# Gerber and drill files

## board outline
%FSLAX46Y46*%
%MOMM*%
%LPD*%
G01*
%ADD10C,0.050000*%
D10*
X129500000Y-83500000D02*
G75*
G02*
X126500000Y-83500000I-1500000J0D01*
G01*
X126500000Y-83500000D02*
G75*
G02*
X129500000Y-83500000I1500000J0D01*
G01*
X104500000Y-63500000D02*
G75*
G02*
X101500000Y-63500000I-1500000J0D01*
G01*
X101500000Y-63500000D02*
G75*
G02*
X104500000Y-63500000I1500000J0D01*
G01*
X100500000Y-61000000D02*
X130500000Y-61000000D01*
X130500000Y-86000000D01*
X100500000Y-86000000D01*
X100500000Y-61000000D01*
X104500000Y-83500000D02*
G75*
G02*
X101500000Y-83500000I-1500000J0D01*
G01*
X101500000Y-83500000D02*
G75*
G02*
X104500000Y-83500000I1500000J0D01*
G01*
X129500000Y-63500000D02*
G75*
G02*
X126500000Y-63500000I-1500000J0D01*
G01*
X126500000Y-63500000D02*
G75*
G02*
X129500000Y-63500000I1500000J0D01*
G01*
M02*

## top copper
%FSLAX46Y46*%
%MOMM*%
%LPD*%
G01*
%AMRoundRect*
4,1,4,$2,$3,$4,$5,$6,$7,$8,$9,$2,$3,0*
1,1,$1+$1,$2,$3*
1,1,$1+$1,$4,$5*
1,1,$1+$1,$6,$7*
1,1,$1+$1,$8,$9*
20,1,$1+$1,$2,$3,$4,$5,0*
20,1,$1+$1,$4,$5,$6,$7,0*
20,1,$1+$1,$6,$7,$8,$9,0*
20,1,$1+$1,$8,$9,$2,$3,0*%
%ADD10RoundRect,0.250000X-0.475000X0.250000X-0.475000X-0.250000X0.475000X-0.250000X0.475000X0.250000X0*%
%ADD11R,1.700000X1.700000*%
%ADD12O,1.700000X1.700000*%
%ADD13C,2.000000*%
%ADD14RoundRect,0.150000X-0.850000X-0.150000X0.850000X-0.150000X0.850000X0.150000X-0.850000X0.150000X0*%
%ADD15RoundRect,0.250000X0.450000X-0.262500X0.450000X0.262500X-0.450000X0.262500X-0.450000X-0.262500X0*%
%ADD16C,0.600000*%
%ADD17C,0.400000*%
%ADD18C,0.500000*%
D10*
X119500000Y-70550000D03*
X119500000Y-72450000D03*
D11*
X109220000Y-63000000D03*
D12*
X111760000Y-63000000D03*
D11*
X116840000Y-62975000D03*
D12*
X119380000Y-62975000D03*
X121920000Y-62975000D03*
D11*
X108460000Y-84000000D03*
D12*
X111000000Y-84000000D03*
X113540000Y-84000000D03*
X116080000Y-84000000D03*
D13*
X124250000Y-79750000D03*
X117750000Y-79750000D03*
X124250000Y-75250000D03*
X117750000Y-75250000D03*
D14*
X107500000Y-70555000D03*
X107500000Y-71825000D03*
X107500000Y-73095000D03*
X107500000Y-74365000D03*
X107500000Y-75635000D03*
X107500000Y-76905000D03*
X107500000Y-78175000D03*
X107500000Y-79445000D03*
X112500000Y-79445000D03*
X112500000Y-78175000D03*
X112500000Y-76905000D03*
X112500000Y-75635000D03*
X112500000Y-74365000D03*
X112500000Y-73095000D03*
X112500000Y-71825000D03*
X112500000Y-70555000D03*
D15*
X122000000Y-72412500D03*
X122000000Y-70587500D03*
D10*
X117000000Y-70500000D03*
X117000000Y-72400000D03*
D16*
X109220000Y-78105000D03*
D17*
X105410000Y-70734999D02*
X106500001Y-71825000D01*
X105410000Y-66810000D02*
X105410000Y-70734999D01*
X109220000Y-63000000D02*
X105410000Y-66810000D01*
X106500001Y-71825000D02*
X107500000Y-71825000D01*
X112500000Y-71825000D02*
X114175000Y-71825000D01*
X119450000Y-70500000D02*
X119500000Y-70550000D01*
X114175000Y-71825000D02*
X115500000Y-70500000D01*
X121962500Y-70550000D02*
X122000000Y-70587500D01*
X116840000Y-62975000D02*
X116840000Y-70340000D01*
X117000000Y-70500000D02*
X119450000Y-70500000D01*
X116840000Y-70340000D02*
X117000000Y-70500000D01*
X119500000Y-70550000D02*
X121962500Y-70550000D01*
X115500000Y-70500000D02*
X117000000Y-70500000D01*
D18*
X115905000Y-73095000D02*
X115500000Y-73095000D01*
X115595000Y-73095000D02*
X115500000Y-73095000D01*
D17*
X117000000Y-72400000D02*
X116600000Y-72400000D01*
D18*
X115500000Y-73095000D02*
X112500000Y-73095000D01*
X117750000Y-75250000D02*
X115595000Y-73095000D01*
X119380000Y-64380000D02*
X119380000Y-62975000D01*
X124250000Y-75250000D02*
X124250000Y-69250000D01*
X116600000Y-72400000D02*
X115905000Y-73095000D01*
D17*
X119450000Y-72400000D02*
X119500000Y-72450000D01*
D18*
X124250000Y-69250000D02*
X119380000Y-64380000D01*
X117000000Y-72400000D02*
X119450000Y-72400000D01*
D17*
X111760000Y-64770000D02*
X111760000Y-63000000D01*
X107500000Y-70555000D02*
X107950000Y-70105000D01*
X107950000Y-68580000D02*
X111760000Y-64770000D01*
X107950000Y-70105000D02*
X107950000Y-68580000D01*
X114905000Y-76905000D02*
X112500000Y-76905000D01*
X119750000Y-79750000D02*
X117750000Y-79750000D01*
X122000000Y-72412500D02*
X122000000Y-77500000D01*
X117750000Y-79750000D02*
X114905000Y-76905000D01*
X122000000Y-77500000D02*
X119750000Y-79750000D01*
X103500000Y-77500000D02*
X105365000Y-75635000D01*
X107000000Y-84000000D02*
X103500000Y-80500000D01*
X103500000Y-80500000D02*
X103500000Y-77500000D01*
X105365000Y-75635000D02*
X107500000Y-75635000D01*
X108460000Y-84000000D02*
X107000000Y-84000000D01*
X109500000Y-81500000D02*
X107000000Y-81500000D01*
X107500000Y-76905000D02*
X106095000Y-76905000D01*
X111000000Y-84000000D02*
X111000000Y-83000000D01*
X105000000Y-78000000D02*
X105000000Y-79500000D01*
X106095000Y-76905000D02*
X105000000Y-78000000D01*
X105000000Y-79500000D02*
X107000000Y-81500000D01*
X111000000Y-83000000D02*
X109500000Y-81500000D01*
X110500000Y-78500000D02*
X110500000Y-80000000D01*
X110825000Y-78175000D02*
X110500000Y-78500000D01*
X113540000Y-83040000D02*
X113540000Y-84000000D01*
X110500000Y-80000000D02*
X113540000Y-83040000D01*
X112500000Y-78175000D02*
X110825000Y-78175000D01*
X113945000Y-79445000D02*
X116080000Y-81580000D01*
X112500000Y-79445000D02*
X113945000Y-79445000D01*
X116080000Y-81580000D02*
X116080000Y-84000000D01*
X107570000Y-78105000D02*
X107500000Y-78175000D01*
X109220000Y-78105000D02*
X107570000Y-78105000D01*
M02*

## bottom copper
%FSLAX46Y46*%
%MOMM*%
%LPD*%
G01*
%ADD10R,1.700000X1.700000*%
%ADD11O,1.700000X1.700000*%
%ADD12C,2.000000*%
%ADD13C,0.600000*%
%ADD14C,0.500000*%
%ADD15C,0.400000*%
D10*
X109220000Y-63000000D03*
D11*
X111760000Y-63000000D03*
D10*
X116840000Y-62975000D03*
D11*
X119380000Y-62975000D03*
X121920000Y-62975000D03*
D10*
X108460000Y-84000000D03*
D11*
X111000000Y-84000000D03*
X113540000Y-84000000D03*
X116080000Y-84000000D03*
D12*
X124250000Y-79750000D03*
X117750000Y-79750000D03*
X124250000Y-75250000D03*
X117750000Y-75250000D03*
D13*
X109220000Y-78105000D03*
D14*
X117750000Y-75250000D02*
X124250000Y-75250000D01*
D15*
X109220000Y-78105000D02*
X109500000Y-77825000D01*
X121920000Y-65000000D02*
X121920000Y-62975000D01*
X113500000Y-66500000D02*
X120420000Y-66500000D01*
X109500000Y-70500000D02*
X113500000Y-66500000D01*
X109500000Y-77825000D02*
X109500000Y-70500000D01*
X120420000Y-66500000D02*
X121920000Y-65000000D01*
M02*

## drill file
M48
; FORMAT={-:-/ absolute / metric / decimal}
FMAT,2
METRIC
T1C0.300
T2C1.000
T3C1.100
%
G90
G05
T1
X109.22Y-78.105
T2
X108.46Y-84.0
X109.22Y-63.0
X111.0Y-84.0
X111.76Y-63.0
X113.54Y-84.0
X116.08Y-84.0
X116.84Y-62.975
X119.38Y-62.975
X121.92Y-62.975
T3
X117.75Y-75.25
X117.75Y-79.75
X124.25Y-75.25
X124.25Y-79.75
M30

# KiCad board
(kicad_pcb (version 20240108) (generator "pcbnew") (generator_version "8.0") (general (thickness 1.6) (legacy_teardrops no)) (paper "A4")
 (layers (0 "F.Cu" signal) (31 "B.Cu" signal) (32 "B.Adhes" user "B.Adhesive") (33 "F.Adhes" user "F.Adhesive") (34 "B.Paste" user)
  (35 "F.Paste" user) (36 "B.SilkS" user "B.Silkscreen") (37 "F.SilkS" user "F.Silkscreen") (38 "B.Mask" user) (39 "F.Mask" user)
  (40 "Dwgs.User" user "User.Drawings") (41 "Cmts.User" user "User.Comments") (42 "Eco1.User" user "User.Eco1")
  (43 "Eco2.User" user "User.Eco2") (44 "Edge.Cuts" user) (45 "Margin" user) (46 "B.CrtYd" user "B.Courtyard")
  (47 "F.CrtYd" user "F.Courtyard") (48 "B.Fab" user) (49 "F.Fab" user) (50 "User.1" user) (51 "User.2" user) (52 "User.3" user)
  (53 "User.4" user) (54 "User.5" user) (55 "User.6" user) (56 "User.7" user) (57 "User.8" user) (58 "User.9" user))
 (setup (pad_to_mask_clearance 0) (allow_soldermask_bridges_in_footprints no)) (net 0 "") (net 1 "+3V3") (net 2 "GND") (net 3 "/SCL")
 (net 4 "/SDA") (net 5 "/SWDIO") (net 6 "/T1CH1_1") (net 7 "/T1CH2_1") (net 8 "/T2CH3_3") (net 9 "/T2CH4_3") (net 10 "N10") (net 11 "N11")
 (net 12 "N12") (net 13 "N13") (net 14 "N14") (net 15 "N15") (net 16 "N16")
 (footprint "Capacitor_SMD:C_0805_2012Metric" (layer "F.Cu") (at 119.5 71.5 -90)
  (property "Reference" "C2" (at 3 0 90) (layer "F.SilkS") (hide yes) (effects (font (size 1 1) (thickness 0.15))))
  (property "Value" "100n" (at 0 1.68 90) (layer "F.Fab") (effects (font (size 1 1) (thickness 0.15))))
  (pad "1" smd roundrect (at -0.95 0 270) (size 1 1.45) (layers "F.Cu" "F.Paste" "F.Mask") (roundrect_rratio 0.25) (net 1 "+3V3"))
  (pad "2" smd roundrect (at 0.95 0 270) (size 1 1.45) (layers "F.Cu" "F.Paste" "F.Mask") (roundrect_rratio 0.25) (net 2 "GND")))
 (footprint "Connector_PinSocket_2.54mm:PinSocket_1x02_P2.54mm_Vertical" (layer "F.Cu") (at 109.22 63 90)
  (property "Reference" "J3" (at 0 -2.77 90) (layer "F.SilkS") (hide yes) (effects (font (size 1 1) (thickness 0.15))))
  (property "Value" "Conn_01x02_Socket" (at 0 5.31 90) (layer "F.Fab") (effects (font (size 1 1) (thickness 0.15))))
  (pad "1" thru_hole rect (at 0 0 90) (size 1.7 1.7) (drill 1) (layers "*.Cu" "*.Mask") (remove_unused_layers no) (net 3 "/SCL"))
  (pad "2" thru_hole oval (at 0 2.54 90) (size 1.7 1.7) (drill 1) (layers "*.Cu" "*.Mask") (remove_unused_layers no) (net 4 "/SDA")))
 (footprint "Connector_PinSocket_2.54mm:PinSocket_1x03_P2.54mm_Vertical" (layer "F.Cu") (at 116.84 62.975 90)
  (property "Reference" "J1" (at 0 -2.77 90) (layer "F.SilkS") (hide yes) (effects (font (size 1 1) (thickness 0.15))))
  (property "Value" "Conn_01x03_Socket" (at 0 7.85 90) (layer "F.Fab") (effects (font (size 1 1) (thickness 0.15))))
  (pad "1" thru_hole rect (at 0 0 90) (size 1.7 1.7) (drill 1) (layers "*.Cu" "*.Mask") (remove_unused_layers no) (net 1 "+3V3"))
  (pad "2" thru_hole oval (at 0 2.54 90) (size 1.7 1.7) (drill 1) (layers "*.Cu" "*.Mask") (remove_unused_layers no) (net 2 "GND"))
  (pad "3" thru_hole oval (at 0 5.08 90) (size 1.7 1.7) (drill 1) (layers "*.Cu" "*.Mask") (remove_unused_layers no) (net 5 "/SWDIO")))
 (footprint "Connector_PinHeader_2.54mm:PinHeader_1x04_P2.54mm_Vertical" (layer "F.Cu") (at 108.46 84 90)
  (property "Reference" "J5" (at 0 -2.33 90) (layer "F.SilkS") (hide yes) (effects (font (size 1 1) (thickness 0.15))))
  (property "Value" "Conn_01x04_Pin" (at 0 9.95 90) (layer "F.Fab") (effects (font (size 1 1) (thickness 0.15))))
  (pad "1" thru_hole rect (at 0 0 90) (size 1.7 1.7) (drill 1) (layers "*.Cu" "*.Mask") (remove_unused_layers no) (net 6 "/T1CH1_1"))
  (pad "2" thru_hole oval (at 0 2.54 90) (size 1.7 1.7) (drill 1) (layers "*.Cu" "*.Mask") (remove_unused_layers no) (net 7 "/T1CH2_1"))
  (pad "3" thru_hole oval (at 0 5.08 90) (size 1.7 1.7) (drill 1) (layers "*.Cu" "*.Mask") (remove_unused_layers no) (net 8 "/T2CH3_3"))
  (pad "4" thru_hole oval (at 0 7.62 90) (size 1.7 1.7) (drill 1) (layers "*.Cu" "*.Mask") (remove_unused_layers no) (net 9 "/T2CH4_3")))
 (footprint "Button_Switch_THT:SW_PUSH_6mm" (layer "F.Cu") (at 124.25 79.75 180)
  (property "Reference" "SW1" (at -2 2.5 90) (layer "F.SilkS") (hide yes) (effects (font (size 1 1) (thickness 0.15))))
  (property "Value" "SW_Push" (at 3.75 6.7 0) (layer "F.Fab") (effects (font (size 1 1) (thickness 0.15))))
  (pad "1" thru_hole circle (at 0 0 270) (size 2 2) (drill 1.1) (layers "*.Cu" "*.Mask") (remove_unused_layers no) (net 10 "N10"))
  (pad "1" thru_hole circle (at 6.5 0 270) (size 2 2) (drill 1.1) (layers "*.Cu" "*.Mask") (remove_unused_layers no) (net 10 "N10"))
  (pad "2" thru_hole circle (at 0 4.5 270) (size 2 2) (drill 1.1) (layers "*.Cu" "*.Mask") (remove_unused_layers no) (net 2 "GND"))
  (pad "2" thru_hole circle (at 6.5 4.5 270) (size 2 2) (drill 1.1) (layers "*.Cu" "*.Mask") (remove_unused_layers no) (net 2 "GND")))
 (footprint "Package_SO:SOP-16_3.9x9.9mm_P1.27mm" (layer "F.Cu") (at 110 75)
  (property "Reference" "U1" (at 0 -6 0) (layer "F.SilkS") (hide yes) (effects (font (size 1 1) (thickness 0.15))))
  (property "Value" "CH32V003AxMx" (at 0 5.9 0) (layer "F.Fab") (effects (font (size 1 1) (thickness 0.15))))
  (pad "1" smd roundrect (at -2.5 -4.445) (size 2 0.6) (layers "F.Cu" "F.Paste" "F.Mask") (roundrect_rratio 0.25) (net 4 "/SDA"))
  (pad "2" smd roundrect (at -2.5 -3.175) (size 2 0.6) (layers "F.Cu" "F.Paste" "F.Mask") (roundrect_rratio 0.25) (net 3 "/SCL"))
  (pad "3" smd roundrect (at -2.5 -1.905) (size 2 0.6) (layers "F.Cu" "F.Paste" "F.Mask") (roundrect_rratio 0.25) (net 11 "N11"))
  (pad "4" smd roundrect (at -2.5 -0.635) (size 2 0.6) (layers "F.Cu" "F.Paste" "F.Mask") (roundrect_rratio 0.25) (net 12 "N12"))
  (pad "5" smd roundrect (at -2.5 0.635) (size 2 0.6) (layers "F.Cu" "F.Paste" "F.Mask") (roundrect_rratio 0.25) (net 6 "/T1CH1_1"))
  (pad "6" smd roundrect (at -2.5 1.905) (size 2 0.6) (layers "F.Cu" "F.Paste" "F.Mask") (roundrect_rratio 0.25) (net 7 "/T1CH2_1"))
  (pad "7" smd roundrect (at -2.5 3.175) (size 2 0.6) (layers "F.Cu" "F.Paste" "F.Mask") (roundrect_rratio 0.25) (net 5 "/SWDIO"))
  (pad "8" smd roundrect (at -2.5 4.445) (size 2 0.6) (layers "F.Cu" "F.Paste" "F.Mask") (roundrect_rratio 0.25) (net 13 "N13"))
  (pad "9" smd roundrect (at 2.5 4.445) (size 2 0.6) (layers "F.Cu" "F.Paste" "F.Mask") (roundrect_rratio 0.25) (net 9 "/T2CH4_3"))
  (pad "10" smd roundrect (at 2.5 3.175) (size 2 0.6) (layers "F.Cu" "F.Paste" "F.Mask") (roundrect_rratio 0.25) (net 8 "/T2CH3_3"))
  (pad "11" smd roundrect (at 2.5 1.905) (size 2 0.6) (layers "F.Cu" "F.Paste" "F.Mask") (roundrect_rratio 0.25) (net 10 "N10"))
  (pad "12" smd roundrect (at 2.5 0.635) (size 2 0.6) (layers "F.Cu" "F.Paste" "F.Mask") (roundrect_rratio 0.25) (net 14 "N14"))
  (pad "13" smd roundrect (at 2.5 -0.635) (size 2 0.6) (layers "F.Cu" "F.Paste" "F.Mask") (roundrect_rratio 0.25) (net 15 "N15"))
  (pad "14" smd roundrect (at 2.5 -1.905) (size 2 0.6) (layers "F.Cu" "F.Paste" "F.Mask") (roundrect_rratio 0.25) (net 2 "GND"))
  (pad "15" smd roundrect (at 2.5 -3.175) (size 2 0.6) (layers "F.Cu" "F.Paste" "F.Mask") (roundrect_rratio 0.25) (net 1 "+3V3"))
  (pad "16" smd roundrect (at 2.5 -4.445) (size 2 0.6) (layers "F.Cu" "F.Paste" "F.Mask") (roundrect_rratio 0.25) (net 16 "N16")))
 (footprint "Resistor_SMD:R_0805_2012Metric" (layer "F.Cu") (at 122 71.5 90)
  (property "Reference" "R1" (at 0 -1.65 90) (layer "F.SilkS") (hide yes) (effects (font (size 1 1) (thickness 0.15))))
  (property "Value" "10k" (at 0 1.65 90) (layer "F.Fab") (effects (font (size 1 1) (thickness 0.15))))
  (pad "1" smd roundrect (at -0.9125 0 90) (size 1.025 1.4) (layers "F.Cu" "F.Paste" "F.Mask") (roundrect_rratio 0.243902) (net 10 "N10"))
  (pad "2" smd roundrect (at 0.9125 0 90) (size 1.025 1.4) (layers "F.Cu" "F.Paste" "F.Mask") (roundrect_rratio 0.243902) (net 1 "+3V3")))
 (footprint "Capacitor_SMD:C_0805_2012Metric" (layer "F.Cu") (at 117 71.45 -90)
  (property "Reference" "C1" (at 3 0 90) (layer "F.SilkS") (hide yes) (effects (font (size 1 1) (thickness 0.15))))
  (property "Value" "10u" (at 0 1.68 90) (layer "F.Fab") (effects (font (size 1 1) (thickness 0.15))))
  (pad "1" smd roundrect (at -0.95 0 270) (size 1 1.45) (layers "F.Cu" "F.Paste" "F.Mask") (roundrect_rratio 0.25) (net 1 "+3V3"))
  (pad "2" smd roundrect (at 0.95 0 270) (size 1 1.45) (layers "F.Cu" "F.Paste" "F.Mask") (roundrect_rratio 0.25) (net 2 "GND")))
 (gr_circle (center 128 83.5) (end 126.5 83.5) (stroke (width 0.05) (type default)) (fill none) (layer "Edge.Cuts"))
 (gr_circle (center 103 63.5) (end 104.5 63.5) (stroke (width 0.05) (type default)) (fill none) (layer "Edge.Cuts"))
 (gr_rect (start 100.5 61) (end 130.5 86) (stroke (width 0.05) (type default)) (fill none) (layer "Edge.Cuts"))
 (gr_circle (center 103 83.5) (end 104.5 83.5) (stroke (width 0.05) (type default)) (fill none) (layer "Edge.Cuts"))
 (gr_circle (center 128 63.5) (end 126.5 63.5) (stroke (width 0.05) (type default)) (fill none) (layer "Edge.Cuts"))
 (segment (start 105.41 70.734999) (end 106.500001 71.825) (width 0.4) (layer "F.Cu") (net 3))
 (segment (start 105.41 66.81) (end 105.41 70.734999) (width 0.4) (layer "F.Cu") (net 3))
 (segment (start 109.22 63) (end 105.41 66.81) (width 0.4) (layer "F.Cu") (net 3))
 (segment (start 106.500001 71.825) (end 107.5 71.825) (width 0.4) (layer "F.Cu") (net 3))
 (segment (start 112.5 71.825) (end 114.175 71.825) (width 0.4) (layer "F.Cu") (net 1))
 (segment (start 119.45 70.5) (end 119.5 70.55) (width 0.4) (layer "F.Cu") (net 1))
 (segment (start 114.175 71.825) (end 115.5 70.5) (width 0.4) (layer "F.Cu") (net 1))
 (segment (start 121.9625 70.55) (end 122 70.5875) (width 0.4) (layer "F.Cu") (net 1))
 (segment (start 116.84 62.975) (end 116.84 70.34) (width 0.4) (layer "F.Cu") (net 1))
 (segment (start 117 70.5) (end 119.45 70.5) (width 0.4) (layer "F.Cu") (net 1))
 (segment (start 116.84 70.34) (end 117 70.5) (width 0.4) (layer "F.Cu") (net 1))
 (segment (start 119.5 70.55) (end 121.9625 70.55) (width 0.4) (layer "F.Cu") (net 1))
 (segment (start 115.5 70.5) (end 117 70.5) (width 0.4) (layer "F.Cu") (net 1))
 (segment (start 115.905 73.095) (end 115.5 73.095) (width 0.5) (layer "F.Cu") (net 2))
 (segment (start 115.595 73.095) (end 115.5 73.095) (width 0.5) (layer "F.Cu") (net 2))
 (segment (start 117 72.4) (end 116.6 72.4) (width 0.4) (layer "F.Cu") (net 2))
 (segment (start 115.5 73.095) (end 112.5 73.095) (width 0.5) (layer "F.Cu") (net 2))
 (segment (start 117.75 75.25) (end 115.595 73.095) (width 0.5) (layer "F.Cu") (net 2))
 (segment (start 119.38 64.38) (end 119.38 62.975) (width 0.5) (layer "F.Cu") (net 2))
 (segment (start 124.25 75.25) (end 124.25 69.25) (width 0.5) (layer "F.Cu") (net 2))
 (segment (start 116.6 72.4) (end 115.905 73.095) (width 0.5) (layer "F.Cu") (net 2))
 (segment (start 119.45 72.4) (end 119.5 72.45) (width 0.4) (layer "F.Cu") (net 2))
 (segment (start 124.25 69.25) (end 119.38 64.38) (width 0.5) (layer "F.Cu") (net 2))
 (segment (start 117 72.4) (end 119.45 72.4) (width 0.5) (layer "F.Cu") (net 2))
 (segment (start 117.75 75.25) (end 124.25 75.25) (width 0.5) (layer "B.Cu") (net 2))
 (segment (start 111.76 64.77) (end 111.76 63) (width 0.4) (layer "F.Cu") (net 4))
 (segment (start 107.5 70.555) (end 107.95 70.105) (width 0.4) (layer "F.Cu") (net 4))
 (segment (start 107.95 68.58) (end 111.76 64.77) (width 0.4) (layer "F.Cu") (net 4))
 (segment (start 107.95 70.105) (end 107.95 68.58) (width 0.4) (layer "F.Cu") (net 4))
 (segment (start 114.905 76.905) (end 112.5 76.905) (width 0.4) (layer "F.Cu") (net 10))
 (segment (start 119.75 79.75) (end 117.75 79.75) (width 0.4) (layer "F.Cu") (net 10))
 (segment (start 122 72.4125) (end 122 77.5) (width 0.4) (layer "F.Cu") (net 10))
 (segment (start 117.75 79.75) (end 114.905 76.905) (width 0.4) (layer "F.Cu") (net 10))
 (segment (start 122 77.5) (end 119.75 79.75) (width 0.4) (layer "F.Cu") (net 10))
 (segment (start 103.5 77.5) (end 105.365 75.635) (width 0.4) (layer "F.Cu") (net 6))
 (segment (start 107 84) (end 103.5 80.5) (width 0.4) (layer "F.Cu") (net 6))
 (segment (start 103.5 80.5) (end 103.5 77.5) (width 0.4) (layer "F.Cu") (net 6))
 (segment (start 105.365 75.635) (end 107.5 75.635) (width 0.4) (layer "F.Cu") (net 6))
 (segment (start 108.46 84) (end 107 84) (width 0.4) (layer "F.Cu") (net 6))
 (segment (start 109.5 81.5) (end 107 81.5) (width 0.4) (layer "F.Cu") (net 7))
 (segment (start 107.5 76.905) (end 106.095 76.905) (width 0.4) (layer "F.Cu") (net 7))
 (segment (start 111 84) (end 111 83) (width 0.4) (layer "F.Cu") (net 7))
 (segment (start 105 78) (end 105 79.5) (width 0.4) (layer "F.Cu") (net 7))
 (segment (start 106.095 76.905) (end 105 78) (width 0.4) (layer "F.Cu") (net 7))
 (segment (start 105 79.5) (end 107 81.5) (width 0.4) (layer "F.Cu") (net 7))
 (segment (start 111 83) (end 109.5 81.5) (width 0.4) (layer "F.Cu") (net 7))
 (segment (start 110.5 78.5) (end 110.5 80) (width 0.4) (layer "F.Cu") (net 8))
 (segment (start 110.825 78.175) (end 110.5 78.5) (width 0.4) (layer "F.Cu") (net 8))
 (segment (start 113.54 83.04) (end 113.54 84) (width 0.4) (layer "F.Cu") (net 8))
 (segment (start 110.5 80) (end 113.54 83.04) (width 0.4) (layer "F.Cu") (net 8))
 (segment (start 112.5 78.175) (end 110.825 78.175) (width 0.4) (layer "F.Cu") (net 8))
 (segment (start 113.945 79.445) (end 116.08 81.58) (width 0.4) (layer "F.Cu") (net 9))
 (segment (start 112.5 79.445) (end 113.945 79.445) (width 0.4) (layer "F.Cu") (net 9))
 (segment (start 116.08 81.58) (end 116.08 84) (width 0.4) (layer "F.Cu") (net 9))
 (segment (start 107.57 78.105) (end 107.5 78.175) (width 0.4) (layer "F.Cu") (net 5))
 (segment (start 109.22 78.105) (end 107.57 78.105) (width 0.4) (layer "F.Cu") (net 5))
 (via (at 109.22 78.105) (size 0.6) (drill 0.3) (layers "F.Cu" "B.Cu") (free yes) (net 5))
 (segment (start 109.22 78.105) (end 109.5 77.825) (width 0.4) (layer "B.Cu") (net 5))
 (segment (start 121.92 65) (end 121.92 62.975) (width 0.4) (layer "B.Cu") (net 5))
 (segment (start 113.5 66.5) (end 120.42 66.5) (width 0.4) (layer "B.Cu") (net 5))
 (segment (start 109.5 70.5) (end 113.5 66.5) (width 0.4) (layer "B.Cu") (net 5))
 (segment (start 109.5 77.825) (end 109.5 70.5) (width 0.4) (layer "B.Cu") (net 5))
 (segment (start 120.42 66.5) (end 121.92 65) (width 0.4) (layer "B.Cu") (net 5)))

